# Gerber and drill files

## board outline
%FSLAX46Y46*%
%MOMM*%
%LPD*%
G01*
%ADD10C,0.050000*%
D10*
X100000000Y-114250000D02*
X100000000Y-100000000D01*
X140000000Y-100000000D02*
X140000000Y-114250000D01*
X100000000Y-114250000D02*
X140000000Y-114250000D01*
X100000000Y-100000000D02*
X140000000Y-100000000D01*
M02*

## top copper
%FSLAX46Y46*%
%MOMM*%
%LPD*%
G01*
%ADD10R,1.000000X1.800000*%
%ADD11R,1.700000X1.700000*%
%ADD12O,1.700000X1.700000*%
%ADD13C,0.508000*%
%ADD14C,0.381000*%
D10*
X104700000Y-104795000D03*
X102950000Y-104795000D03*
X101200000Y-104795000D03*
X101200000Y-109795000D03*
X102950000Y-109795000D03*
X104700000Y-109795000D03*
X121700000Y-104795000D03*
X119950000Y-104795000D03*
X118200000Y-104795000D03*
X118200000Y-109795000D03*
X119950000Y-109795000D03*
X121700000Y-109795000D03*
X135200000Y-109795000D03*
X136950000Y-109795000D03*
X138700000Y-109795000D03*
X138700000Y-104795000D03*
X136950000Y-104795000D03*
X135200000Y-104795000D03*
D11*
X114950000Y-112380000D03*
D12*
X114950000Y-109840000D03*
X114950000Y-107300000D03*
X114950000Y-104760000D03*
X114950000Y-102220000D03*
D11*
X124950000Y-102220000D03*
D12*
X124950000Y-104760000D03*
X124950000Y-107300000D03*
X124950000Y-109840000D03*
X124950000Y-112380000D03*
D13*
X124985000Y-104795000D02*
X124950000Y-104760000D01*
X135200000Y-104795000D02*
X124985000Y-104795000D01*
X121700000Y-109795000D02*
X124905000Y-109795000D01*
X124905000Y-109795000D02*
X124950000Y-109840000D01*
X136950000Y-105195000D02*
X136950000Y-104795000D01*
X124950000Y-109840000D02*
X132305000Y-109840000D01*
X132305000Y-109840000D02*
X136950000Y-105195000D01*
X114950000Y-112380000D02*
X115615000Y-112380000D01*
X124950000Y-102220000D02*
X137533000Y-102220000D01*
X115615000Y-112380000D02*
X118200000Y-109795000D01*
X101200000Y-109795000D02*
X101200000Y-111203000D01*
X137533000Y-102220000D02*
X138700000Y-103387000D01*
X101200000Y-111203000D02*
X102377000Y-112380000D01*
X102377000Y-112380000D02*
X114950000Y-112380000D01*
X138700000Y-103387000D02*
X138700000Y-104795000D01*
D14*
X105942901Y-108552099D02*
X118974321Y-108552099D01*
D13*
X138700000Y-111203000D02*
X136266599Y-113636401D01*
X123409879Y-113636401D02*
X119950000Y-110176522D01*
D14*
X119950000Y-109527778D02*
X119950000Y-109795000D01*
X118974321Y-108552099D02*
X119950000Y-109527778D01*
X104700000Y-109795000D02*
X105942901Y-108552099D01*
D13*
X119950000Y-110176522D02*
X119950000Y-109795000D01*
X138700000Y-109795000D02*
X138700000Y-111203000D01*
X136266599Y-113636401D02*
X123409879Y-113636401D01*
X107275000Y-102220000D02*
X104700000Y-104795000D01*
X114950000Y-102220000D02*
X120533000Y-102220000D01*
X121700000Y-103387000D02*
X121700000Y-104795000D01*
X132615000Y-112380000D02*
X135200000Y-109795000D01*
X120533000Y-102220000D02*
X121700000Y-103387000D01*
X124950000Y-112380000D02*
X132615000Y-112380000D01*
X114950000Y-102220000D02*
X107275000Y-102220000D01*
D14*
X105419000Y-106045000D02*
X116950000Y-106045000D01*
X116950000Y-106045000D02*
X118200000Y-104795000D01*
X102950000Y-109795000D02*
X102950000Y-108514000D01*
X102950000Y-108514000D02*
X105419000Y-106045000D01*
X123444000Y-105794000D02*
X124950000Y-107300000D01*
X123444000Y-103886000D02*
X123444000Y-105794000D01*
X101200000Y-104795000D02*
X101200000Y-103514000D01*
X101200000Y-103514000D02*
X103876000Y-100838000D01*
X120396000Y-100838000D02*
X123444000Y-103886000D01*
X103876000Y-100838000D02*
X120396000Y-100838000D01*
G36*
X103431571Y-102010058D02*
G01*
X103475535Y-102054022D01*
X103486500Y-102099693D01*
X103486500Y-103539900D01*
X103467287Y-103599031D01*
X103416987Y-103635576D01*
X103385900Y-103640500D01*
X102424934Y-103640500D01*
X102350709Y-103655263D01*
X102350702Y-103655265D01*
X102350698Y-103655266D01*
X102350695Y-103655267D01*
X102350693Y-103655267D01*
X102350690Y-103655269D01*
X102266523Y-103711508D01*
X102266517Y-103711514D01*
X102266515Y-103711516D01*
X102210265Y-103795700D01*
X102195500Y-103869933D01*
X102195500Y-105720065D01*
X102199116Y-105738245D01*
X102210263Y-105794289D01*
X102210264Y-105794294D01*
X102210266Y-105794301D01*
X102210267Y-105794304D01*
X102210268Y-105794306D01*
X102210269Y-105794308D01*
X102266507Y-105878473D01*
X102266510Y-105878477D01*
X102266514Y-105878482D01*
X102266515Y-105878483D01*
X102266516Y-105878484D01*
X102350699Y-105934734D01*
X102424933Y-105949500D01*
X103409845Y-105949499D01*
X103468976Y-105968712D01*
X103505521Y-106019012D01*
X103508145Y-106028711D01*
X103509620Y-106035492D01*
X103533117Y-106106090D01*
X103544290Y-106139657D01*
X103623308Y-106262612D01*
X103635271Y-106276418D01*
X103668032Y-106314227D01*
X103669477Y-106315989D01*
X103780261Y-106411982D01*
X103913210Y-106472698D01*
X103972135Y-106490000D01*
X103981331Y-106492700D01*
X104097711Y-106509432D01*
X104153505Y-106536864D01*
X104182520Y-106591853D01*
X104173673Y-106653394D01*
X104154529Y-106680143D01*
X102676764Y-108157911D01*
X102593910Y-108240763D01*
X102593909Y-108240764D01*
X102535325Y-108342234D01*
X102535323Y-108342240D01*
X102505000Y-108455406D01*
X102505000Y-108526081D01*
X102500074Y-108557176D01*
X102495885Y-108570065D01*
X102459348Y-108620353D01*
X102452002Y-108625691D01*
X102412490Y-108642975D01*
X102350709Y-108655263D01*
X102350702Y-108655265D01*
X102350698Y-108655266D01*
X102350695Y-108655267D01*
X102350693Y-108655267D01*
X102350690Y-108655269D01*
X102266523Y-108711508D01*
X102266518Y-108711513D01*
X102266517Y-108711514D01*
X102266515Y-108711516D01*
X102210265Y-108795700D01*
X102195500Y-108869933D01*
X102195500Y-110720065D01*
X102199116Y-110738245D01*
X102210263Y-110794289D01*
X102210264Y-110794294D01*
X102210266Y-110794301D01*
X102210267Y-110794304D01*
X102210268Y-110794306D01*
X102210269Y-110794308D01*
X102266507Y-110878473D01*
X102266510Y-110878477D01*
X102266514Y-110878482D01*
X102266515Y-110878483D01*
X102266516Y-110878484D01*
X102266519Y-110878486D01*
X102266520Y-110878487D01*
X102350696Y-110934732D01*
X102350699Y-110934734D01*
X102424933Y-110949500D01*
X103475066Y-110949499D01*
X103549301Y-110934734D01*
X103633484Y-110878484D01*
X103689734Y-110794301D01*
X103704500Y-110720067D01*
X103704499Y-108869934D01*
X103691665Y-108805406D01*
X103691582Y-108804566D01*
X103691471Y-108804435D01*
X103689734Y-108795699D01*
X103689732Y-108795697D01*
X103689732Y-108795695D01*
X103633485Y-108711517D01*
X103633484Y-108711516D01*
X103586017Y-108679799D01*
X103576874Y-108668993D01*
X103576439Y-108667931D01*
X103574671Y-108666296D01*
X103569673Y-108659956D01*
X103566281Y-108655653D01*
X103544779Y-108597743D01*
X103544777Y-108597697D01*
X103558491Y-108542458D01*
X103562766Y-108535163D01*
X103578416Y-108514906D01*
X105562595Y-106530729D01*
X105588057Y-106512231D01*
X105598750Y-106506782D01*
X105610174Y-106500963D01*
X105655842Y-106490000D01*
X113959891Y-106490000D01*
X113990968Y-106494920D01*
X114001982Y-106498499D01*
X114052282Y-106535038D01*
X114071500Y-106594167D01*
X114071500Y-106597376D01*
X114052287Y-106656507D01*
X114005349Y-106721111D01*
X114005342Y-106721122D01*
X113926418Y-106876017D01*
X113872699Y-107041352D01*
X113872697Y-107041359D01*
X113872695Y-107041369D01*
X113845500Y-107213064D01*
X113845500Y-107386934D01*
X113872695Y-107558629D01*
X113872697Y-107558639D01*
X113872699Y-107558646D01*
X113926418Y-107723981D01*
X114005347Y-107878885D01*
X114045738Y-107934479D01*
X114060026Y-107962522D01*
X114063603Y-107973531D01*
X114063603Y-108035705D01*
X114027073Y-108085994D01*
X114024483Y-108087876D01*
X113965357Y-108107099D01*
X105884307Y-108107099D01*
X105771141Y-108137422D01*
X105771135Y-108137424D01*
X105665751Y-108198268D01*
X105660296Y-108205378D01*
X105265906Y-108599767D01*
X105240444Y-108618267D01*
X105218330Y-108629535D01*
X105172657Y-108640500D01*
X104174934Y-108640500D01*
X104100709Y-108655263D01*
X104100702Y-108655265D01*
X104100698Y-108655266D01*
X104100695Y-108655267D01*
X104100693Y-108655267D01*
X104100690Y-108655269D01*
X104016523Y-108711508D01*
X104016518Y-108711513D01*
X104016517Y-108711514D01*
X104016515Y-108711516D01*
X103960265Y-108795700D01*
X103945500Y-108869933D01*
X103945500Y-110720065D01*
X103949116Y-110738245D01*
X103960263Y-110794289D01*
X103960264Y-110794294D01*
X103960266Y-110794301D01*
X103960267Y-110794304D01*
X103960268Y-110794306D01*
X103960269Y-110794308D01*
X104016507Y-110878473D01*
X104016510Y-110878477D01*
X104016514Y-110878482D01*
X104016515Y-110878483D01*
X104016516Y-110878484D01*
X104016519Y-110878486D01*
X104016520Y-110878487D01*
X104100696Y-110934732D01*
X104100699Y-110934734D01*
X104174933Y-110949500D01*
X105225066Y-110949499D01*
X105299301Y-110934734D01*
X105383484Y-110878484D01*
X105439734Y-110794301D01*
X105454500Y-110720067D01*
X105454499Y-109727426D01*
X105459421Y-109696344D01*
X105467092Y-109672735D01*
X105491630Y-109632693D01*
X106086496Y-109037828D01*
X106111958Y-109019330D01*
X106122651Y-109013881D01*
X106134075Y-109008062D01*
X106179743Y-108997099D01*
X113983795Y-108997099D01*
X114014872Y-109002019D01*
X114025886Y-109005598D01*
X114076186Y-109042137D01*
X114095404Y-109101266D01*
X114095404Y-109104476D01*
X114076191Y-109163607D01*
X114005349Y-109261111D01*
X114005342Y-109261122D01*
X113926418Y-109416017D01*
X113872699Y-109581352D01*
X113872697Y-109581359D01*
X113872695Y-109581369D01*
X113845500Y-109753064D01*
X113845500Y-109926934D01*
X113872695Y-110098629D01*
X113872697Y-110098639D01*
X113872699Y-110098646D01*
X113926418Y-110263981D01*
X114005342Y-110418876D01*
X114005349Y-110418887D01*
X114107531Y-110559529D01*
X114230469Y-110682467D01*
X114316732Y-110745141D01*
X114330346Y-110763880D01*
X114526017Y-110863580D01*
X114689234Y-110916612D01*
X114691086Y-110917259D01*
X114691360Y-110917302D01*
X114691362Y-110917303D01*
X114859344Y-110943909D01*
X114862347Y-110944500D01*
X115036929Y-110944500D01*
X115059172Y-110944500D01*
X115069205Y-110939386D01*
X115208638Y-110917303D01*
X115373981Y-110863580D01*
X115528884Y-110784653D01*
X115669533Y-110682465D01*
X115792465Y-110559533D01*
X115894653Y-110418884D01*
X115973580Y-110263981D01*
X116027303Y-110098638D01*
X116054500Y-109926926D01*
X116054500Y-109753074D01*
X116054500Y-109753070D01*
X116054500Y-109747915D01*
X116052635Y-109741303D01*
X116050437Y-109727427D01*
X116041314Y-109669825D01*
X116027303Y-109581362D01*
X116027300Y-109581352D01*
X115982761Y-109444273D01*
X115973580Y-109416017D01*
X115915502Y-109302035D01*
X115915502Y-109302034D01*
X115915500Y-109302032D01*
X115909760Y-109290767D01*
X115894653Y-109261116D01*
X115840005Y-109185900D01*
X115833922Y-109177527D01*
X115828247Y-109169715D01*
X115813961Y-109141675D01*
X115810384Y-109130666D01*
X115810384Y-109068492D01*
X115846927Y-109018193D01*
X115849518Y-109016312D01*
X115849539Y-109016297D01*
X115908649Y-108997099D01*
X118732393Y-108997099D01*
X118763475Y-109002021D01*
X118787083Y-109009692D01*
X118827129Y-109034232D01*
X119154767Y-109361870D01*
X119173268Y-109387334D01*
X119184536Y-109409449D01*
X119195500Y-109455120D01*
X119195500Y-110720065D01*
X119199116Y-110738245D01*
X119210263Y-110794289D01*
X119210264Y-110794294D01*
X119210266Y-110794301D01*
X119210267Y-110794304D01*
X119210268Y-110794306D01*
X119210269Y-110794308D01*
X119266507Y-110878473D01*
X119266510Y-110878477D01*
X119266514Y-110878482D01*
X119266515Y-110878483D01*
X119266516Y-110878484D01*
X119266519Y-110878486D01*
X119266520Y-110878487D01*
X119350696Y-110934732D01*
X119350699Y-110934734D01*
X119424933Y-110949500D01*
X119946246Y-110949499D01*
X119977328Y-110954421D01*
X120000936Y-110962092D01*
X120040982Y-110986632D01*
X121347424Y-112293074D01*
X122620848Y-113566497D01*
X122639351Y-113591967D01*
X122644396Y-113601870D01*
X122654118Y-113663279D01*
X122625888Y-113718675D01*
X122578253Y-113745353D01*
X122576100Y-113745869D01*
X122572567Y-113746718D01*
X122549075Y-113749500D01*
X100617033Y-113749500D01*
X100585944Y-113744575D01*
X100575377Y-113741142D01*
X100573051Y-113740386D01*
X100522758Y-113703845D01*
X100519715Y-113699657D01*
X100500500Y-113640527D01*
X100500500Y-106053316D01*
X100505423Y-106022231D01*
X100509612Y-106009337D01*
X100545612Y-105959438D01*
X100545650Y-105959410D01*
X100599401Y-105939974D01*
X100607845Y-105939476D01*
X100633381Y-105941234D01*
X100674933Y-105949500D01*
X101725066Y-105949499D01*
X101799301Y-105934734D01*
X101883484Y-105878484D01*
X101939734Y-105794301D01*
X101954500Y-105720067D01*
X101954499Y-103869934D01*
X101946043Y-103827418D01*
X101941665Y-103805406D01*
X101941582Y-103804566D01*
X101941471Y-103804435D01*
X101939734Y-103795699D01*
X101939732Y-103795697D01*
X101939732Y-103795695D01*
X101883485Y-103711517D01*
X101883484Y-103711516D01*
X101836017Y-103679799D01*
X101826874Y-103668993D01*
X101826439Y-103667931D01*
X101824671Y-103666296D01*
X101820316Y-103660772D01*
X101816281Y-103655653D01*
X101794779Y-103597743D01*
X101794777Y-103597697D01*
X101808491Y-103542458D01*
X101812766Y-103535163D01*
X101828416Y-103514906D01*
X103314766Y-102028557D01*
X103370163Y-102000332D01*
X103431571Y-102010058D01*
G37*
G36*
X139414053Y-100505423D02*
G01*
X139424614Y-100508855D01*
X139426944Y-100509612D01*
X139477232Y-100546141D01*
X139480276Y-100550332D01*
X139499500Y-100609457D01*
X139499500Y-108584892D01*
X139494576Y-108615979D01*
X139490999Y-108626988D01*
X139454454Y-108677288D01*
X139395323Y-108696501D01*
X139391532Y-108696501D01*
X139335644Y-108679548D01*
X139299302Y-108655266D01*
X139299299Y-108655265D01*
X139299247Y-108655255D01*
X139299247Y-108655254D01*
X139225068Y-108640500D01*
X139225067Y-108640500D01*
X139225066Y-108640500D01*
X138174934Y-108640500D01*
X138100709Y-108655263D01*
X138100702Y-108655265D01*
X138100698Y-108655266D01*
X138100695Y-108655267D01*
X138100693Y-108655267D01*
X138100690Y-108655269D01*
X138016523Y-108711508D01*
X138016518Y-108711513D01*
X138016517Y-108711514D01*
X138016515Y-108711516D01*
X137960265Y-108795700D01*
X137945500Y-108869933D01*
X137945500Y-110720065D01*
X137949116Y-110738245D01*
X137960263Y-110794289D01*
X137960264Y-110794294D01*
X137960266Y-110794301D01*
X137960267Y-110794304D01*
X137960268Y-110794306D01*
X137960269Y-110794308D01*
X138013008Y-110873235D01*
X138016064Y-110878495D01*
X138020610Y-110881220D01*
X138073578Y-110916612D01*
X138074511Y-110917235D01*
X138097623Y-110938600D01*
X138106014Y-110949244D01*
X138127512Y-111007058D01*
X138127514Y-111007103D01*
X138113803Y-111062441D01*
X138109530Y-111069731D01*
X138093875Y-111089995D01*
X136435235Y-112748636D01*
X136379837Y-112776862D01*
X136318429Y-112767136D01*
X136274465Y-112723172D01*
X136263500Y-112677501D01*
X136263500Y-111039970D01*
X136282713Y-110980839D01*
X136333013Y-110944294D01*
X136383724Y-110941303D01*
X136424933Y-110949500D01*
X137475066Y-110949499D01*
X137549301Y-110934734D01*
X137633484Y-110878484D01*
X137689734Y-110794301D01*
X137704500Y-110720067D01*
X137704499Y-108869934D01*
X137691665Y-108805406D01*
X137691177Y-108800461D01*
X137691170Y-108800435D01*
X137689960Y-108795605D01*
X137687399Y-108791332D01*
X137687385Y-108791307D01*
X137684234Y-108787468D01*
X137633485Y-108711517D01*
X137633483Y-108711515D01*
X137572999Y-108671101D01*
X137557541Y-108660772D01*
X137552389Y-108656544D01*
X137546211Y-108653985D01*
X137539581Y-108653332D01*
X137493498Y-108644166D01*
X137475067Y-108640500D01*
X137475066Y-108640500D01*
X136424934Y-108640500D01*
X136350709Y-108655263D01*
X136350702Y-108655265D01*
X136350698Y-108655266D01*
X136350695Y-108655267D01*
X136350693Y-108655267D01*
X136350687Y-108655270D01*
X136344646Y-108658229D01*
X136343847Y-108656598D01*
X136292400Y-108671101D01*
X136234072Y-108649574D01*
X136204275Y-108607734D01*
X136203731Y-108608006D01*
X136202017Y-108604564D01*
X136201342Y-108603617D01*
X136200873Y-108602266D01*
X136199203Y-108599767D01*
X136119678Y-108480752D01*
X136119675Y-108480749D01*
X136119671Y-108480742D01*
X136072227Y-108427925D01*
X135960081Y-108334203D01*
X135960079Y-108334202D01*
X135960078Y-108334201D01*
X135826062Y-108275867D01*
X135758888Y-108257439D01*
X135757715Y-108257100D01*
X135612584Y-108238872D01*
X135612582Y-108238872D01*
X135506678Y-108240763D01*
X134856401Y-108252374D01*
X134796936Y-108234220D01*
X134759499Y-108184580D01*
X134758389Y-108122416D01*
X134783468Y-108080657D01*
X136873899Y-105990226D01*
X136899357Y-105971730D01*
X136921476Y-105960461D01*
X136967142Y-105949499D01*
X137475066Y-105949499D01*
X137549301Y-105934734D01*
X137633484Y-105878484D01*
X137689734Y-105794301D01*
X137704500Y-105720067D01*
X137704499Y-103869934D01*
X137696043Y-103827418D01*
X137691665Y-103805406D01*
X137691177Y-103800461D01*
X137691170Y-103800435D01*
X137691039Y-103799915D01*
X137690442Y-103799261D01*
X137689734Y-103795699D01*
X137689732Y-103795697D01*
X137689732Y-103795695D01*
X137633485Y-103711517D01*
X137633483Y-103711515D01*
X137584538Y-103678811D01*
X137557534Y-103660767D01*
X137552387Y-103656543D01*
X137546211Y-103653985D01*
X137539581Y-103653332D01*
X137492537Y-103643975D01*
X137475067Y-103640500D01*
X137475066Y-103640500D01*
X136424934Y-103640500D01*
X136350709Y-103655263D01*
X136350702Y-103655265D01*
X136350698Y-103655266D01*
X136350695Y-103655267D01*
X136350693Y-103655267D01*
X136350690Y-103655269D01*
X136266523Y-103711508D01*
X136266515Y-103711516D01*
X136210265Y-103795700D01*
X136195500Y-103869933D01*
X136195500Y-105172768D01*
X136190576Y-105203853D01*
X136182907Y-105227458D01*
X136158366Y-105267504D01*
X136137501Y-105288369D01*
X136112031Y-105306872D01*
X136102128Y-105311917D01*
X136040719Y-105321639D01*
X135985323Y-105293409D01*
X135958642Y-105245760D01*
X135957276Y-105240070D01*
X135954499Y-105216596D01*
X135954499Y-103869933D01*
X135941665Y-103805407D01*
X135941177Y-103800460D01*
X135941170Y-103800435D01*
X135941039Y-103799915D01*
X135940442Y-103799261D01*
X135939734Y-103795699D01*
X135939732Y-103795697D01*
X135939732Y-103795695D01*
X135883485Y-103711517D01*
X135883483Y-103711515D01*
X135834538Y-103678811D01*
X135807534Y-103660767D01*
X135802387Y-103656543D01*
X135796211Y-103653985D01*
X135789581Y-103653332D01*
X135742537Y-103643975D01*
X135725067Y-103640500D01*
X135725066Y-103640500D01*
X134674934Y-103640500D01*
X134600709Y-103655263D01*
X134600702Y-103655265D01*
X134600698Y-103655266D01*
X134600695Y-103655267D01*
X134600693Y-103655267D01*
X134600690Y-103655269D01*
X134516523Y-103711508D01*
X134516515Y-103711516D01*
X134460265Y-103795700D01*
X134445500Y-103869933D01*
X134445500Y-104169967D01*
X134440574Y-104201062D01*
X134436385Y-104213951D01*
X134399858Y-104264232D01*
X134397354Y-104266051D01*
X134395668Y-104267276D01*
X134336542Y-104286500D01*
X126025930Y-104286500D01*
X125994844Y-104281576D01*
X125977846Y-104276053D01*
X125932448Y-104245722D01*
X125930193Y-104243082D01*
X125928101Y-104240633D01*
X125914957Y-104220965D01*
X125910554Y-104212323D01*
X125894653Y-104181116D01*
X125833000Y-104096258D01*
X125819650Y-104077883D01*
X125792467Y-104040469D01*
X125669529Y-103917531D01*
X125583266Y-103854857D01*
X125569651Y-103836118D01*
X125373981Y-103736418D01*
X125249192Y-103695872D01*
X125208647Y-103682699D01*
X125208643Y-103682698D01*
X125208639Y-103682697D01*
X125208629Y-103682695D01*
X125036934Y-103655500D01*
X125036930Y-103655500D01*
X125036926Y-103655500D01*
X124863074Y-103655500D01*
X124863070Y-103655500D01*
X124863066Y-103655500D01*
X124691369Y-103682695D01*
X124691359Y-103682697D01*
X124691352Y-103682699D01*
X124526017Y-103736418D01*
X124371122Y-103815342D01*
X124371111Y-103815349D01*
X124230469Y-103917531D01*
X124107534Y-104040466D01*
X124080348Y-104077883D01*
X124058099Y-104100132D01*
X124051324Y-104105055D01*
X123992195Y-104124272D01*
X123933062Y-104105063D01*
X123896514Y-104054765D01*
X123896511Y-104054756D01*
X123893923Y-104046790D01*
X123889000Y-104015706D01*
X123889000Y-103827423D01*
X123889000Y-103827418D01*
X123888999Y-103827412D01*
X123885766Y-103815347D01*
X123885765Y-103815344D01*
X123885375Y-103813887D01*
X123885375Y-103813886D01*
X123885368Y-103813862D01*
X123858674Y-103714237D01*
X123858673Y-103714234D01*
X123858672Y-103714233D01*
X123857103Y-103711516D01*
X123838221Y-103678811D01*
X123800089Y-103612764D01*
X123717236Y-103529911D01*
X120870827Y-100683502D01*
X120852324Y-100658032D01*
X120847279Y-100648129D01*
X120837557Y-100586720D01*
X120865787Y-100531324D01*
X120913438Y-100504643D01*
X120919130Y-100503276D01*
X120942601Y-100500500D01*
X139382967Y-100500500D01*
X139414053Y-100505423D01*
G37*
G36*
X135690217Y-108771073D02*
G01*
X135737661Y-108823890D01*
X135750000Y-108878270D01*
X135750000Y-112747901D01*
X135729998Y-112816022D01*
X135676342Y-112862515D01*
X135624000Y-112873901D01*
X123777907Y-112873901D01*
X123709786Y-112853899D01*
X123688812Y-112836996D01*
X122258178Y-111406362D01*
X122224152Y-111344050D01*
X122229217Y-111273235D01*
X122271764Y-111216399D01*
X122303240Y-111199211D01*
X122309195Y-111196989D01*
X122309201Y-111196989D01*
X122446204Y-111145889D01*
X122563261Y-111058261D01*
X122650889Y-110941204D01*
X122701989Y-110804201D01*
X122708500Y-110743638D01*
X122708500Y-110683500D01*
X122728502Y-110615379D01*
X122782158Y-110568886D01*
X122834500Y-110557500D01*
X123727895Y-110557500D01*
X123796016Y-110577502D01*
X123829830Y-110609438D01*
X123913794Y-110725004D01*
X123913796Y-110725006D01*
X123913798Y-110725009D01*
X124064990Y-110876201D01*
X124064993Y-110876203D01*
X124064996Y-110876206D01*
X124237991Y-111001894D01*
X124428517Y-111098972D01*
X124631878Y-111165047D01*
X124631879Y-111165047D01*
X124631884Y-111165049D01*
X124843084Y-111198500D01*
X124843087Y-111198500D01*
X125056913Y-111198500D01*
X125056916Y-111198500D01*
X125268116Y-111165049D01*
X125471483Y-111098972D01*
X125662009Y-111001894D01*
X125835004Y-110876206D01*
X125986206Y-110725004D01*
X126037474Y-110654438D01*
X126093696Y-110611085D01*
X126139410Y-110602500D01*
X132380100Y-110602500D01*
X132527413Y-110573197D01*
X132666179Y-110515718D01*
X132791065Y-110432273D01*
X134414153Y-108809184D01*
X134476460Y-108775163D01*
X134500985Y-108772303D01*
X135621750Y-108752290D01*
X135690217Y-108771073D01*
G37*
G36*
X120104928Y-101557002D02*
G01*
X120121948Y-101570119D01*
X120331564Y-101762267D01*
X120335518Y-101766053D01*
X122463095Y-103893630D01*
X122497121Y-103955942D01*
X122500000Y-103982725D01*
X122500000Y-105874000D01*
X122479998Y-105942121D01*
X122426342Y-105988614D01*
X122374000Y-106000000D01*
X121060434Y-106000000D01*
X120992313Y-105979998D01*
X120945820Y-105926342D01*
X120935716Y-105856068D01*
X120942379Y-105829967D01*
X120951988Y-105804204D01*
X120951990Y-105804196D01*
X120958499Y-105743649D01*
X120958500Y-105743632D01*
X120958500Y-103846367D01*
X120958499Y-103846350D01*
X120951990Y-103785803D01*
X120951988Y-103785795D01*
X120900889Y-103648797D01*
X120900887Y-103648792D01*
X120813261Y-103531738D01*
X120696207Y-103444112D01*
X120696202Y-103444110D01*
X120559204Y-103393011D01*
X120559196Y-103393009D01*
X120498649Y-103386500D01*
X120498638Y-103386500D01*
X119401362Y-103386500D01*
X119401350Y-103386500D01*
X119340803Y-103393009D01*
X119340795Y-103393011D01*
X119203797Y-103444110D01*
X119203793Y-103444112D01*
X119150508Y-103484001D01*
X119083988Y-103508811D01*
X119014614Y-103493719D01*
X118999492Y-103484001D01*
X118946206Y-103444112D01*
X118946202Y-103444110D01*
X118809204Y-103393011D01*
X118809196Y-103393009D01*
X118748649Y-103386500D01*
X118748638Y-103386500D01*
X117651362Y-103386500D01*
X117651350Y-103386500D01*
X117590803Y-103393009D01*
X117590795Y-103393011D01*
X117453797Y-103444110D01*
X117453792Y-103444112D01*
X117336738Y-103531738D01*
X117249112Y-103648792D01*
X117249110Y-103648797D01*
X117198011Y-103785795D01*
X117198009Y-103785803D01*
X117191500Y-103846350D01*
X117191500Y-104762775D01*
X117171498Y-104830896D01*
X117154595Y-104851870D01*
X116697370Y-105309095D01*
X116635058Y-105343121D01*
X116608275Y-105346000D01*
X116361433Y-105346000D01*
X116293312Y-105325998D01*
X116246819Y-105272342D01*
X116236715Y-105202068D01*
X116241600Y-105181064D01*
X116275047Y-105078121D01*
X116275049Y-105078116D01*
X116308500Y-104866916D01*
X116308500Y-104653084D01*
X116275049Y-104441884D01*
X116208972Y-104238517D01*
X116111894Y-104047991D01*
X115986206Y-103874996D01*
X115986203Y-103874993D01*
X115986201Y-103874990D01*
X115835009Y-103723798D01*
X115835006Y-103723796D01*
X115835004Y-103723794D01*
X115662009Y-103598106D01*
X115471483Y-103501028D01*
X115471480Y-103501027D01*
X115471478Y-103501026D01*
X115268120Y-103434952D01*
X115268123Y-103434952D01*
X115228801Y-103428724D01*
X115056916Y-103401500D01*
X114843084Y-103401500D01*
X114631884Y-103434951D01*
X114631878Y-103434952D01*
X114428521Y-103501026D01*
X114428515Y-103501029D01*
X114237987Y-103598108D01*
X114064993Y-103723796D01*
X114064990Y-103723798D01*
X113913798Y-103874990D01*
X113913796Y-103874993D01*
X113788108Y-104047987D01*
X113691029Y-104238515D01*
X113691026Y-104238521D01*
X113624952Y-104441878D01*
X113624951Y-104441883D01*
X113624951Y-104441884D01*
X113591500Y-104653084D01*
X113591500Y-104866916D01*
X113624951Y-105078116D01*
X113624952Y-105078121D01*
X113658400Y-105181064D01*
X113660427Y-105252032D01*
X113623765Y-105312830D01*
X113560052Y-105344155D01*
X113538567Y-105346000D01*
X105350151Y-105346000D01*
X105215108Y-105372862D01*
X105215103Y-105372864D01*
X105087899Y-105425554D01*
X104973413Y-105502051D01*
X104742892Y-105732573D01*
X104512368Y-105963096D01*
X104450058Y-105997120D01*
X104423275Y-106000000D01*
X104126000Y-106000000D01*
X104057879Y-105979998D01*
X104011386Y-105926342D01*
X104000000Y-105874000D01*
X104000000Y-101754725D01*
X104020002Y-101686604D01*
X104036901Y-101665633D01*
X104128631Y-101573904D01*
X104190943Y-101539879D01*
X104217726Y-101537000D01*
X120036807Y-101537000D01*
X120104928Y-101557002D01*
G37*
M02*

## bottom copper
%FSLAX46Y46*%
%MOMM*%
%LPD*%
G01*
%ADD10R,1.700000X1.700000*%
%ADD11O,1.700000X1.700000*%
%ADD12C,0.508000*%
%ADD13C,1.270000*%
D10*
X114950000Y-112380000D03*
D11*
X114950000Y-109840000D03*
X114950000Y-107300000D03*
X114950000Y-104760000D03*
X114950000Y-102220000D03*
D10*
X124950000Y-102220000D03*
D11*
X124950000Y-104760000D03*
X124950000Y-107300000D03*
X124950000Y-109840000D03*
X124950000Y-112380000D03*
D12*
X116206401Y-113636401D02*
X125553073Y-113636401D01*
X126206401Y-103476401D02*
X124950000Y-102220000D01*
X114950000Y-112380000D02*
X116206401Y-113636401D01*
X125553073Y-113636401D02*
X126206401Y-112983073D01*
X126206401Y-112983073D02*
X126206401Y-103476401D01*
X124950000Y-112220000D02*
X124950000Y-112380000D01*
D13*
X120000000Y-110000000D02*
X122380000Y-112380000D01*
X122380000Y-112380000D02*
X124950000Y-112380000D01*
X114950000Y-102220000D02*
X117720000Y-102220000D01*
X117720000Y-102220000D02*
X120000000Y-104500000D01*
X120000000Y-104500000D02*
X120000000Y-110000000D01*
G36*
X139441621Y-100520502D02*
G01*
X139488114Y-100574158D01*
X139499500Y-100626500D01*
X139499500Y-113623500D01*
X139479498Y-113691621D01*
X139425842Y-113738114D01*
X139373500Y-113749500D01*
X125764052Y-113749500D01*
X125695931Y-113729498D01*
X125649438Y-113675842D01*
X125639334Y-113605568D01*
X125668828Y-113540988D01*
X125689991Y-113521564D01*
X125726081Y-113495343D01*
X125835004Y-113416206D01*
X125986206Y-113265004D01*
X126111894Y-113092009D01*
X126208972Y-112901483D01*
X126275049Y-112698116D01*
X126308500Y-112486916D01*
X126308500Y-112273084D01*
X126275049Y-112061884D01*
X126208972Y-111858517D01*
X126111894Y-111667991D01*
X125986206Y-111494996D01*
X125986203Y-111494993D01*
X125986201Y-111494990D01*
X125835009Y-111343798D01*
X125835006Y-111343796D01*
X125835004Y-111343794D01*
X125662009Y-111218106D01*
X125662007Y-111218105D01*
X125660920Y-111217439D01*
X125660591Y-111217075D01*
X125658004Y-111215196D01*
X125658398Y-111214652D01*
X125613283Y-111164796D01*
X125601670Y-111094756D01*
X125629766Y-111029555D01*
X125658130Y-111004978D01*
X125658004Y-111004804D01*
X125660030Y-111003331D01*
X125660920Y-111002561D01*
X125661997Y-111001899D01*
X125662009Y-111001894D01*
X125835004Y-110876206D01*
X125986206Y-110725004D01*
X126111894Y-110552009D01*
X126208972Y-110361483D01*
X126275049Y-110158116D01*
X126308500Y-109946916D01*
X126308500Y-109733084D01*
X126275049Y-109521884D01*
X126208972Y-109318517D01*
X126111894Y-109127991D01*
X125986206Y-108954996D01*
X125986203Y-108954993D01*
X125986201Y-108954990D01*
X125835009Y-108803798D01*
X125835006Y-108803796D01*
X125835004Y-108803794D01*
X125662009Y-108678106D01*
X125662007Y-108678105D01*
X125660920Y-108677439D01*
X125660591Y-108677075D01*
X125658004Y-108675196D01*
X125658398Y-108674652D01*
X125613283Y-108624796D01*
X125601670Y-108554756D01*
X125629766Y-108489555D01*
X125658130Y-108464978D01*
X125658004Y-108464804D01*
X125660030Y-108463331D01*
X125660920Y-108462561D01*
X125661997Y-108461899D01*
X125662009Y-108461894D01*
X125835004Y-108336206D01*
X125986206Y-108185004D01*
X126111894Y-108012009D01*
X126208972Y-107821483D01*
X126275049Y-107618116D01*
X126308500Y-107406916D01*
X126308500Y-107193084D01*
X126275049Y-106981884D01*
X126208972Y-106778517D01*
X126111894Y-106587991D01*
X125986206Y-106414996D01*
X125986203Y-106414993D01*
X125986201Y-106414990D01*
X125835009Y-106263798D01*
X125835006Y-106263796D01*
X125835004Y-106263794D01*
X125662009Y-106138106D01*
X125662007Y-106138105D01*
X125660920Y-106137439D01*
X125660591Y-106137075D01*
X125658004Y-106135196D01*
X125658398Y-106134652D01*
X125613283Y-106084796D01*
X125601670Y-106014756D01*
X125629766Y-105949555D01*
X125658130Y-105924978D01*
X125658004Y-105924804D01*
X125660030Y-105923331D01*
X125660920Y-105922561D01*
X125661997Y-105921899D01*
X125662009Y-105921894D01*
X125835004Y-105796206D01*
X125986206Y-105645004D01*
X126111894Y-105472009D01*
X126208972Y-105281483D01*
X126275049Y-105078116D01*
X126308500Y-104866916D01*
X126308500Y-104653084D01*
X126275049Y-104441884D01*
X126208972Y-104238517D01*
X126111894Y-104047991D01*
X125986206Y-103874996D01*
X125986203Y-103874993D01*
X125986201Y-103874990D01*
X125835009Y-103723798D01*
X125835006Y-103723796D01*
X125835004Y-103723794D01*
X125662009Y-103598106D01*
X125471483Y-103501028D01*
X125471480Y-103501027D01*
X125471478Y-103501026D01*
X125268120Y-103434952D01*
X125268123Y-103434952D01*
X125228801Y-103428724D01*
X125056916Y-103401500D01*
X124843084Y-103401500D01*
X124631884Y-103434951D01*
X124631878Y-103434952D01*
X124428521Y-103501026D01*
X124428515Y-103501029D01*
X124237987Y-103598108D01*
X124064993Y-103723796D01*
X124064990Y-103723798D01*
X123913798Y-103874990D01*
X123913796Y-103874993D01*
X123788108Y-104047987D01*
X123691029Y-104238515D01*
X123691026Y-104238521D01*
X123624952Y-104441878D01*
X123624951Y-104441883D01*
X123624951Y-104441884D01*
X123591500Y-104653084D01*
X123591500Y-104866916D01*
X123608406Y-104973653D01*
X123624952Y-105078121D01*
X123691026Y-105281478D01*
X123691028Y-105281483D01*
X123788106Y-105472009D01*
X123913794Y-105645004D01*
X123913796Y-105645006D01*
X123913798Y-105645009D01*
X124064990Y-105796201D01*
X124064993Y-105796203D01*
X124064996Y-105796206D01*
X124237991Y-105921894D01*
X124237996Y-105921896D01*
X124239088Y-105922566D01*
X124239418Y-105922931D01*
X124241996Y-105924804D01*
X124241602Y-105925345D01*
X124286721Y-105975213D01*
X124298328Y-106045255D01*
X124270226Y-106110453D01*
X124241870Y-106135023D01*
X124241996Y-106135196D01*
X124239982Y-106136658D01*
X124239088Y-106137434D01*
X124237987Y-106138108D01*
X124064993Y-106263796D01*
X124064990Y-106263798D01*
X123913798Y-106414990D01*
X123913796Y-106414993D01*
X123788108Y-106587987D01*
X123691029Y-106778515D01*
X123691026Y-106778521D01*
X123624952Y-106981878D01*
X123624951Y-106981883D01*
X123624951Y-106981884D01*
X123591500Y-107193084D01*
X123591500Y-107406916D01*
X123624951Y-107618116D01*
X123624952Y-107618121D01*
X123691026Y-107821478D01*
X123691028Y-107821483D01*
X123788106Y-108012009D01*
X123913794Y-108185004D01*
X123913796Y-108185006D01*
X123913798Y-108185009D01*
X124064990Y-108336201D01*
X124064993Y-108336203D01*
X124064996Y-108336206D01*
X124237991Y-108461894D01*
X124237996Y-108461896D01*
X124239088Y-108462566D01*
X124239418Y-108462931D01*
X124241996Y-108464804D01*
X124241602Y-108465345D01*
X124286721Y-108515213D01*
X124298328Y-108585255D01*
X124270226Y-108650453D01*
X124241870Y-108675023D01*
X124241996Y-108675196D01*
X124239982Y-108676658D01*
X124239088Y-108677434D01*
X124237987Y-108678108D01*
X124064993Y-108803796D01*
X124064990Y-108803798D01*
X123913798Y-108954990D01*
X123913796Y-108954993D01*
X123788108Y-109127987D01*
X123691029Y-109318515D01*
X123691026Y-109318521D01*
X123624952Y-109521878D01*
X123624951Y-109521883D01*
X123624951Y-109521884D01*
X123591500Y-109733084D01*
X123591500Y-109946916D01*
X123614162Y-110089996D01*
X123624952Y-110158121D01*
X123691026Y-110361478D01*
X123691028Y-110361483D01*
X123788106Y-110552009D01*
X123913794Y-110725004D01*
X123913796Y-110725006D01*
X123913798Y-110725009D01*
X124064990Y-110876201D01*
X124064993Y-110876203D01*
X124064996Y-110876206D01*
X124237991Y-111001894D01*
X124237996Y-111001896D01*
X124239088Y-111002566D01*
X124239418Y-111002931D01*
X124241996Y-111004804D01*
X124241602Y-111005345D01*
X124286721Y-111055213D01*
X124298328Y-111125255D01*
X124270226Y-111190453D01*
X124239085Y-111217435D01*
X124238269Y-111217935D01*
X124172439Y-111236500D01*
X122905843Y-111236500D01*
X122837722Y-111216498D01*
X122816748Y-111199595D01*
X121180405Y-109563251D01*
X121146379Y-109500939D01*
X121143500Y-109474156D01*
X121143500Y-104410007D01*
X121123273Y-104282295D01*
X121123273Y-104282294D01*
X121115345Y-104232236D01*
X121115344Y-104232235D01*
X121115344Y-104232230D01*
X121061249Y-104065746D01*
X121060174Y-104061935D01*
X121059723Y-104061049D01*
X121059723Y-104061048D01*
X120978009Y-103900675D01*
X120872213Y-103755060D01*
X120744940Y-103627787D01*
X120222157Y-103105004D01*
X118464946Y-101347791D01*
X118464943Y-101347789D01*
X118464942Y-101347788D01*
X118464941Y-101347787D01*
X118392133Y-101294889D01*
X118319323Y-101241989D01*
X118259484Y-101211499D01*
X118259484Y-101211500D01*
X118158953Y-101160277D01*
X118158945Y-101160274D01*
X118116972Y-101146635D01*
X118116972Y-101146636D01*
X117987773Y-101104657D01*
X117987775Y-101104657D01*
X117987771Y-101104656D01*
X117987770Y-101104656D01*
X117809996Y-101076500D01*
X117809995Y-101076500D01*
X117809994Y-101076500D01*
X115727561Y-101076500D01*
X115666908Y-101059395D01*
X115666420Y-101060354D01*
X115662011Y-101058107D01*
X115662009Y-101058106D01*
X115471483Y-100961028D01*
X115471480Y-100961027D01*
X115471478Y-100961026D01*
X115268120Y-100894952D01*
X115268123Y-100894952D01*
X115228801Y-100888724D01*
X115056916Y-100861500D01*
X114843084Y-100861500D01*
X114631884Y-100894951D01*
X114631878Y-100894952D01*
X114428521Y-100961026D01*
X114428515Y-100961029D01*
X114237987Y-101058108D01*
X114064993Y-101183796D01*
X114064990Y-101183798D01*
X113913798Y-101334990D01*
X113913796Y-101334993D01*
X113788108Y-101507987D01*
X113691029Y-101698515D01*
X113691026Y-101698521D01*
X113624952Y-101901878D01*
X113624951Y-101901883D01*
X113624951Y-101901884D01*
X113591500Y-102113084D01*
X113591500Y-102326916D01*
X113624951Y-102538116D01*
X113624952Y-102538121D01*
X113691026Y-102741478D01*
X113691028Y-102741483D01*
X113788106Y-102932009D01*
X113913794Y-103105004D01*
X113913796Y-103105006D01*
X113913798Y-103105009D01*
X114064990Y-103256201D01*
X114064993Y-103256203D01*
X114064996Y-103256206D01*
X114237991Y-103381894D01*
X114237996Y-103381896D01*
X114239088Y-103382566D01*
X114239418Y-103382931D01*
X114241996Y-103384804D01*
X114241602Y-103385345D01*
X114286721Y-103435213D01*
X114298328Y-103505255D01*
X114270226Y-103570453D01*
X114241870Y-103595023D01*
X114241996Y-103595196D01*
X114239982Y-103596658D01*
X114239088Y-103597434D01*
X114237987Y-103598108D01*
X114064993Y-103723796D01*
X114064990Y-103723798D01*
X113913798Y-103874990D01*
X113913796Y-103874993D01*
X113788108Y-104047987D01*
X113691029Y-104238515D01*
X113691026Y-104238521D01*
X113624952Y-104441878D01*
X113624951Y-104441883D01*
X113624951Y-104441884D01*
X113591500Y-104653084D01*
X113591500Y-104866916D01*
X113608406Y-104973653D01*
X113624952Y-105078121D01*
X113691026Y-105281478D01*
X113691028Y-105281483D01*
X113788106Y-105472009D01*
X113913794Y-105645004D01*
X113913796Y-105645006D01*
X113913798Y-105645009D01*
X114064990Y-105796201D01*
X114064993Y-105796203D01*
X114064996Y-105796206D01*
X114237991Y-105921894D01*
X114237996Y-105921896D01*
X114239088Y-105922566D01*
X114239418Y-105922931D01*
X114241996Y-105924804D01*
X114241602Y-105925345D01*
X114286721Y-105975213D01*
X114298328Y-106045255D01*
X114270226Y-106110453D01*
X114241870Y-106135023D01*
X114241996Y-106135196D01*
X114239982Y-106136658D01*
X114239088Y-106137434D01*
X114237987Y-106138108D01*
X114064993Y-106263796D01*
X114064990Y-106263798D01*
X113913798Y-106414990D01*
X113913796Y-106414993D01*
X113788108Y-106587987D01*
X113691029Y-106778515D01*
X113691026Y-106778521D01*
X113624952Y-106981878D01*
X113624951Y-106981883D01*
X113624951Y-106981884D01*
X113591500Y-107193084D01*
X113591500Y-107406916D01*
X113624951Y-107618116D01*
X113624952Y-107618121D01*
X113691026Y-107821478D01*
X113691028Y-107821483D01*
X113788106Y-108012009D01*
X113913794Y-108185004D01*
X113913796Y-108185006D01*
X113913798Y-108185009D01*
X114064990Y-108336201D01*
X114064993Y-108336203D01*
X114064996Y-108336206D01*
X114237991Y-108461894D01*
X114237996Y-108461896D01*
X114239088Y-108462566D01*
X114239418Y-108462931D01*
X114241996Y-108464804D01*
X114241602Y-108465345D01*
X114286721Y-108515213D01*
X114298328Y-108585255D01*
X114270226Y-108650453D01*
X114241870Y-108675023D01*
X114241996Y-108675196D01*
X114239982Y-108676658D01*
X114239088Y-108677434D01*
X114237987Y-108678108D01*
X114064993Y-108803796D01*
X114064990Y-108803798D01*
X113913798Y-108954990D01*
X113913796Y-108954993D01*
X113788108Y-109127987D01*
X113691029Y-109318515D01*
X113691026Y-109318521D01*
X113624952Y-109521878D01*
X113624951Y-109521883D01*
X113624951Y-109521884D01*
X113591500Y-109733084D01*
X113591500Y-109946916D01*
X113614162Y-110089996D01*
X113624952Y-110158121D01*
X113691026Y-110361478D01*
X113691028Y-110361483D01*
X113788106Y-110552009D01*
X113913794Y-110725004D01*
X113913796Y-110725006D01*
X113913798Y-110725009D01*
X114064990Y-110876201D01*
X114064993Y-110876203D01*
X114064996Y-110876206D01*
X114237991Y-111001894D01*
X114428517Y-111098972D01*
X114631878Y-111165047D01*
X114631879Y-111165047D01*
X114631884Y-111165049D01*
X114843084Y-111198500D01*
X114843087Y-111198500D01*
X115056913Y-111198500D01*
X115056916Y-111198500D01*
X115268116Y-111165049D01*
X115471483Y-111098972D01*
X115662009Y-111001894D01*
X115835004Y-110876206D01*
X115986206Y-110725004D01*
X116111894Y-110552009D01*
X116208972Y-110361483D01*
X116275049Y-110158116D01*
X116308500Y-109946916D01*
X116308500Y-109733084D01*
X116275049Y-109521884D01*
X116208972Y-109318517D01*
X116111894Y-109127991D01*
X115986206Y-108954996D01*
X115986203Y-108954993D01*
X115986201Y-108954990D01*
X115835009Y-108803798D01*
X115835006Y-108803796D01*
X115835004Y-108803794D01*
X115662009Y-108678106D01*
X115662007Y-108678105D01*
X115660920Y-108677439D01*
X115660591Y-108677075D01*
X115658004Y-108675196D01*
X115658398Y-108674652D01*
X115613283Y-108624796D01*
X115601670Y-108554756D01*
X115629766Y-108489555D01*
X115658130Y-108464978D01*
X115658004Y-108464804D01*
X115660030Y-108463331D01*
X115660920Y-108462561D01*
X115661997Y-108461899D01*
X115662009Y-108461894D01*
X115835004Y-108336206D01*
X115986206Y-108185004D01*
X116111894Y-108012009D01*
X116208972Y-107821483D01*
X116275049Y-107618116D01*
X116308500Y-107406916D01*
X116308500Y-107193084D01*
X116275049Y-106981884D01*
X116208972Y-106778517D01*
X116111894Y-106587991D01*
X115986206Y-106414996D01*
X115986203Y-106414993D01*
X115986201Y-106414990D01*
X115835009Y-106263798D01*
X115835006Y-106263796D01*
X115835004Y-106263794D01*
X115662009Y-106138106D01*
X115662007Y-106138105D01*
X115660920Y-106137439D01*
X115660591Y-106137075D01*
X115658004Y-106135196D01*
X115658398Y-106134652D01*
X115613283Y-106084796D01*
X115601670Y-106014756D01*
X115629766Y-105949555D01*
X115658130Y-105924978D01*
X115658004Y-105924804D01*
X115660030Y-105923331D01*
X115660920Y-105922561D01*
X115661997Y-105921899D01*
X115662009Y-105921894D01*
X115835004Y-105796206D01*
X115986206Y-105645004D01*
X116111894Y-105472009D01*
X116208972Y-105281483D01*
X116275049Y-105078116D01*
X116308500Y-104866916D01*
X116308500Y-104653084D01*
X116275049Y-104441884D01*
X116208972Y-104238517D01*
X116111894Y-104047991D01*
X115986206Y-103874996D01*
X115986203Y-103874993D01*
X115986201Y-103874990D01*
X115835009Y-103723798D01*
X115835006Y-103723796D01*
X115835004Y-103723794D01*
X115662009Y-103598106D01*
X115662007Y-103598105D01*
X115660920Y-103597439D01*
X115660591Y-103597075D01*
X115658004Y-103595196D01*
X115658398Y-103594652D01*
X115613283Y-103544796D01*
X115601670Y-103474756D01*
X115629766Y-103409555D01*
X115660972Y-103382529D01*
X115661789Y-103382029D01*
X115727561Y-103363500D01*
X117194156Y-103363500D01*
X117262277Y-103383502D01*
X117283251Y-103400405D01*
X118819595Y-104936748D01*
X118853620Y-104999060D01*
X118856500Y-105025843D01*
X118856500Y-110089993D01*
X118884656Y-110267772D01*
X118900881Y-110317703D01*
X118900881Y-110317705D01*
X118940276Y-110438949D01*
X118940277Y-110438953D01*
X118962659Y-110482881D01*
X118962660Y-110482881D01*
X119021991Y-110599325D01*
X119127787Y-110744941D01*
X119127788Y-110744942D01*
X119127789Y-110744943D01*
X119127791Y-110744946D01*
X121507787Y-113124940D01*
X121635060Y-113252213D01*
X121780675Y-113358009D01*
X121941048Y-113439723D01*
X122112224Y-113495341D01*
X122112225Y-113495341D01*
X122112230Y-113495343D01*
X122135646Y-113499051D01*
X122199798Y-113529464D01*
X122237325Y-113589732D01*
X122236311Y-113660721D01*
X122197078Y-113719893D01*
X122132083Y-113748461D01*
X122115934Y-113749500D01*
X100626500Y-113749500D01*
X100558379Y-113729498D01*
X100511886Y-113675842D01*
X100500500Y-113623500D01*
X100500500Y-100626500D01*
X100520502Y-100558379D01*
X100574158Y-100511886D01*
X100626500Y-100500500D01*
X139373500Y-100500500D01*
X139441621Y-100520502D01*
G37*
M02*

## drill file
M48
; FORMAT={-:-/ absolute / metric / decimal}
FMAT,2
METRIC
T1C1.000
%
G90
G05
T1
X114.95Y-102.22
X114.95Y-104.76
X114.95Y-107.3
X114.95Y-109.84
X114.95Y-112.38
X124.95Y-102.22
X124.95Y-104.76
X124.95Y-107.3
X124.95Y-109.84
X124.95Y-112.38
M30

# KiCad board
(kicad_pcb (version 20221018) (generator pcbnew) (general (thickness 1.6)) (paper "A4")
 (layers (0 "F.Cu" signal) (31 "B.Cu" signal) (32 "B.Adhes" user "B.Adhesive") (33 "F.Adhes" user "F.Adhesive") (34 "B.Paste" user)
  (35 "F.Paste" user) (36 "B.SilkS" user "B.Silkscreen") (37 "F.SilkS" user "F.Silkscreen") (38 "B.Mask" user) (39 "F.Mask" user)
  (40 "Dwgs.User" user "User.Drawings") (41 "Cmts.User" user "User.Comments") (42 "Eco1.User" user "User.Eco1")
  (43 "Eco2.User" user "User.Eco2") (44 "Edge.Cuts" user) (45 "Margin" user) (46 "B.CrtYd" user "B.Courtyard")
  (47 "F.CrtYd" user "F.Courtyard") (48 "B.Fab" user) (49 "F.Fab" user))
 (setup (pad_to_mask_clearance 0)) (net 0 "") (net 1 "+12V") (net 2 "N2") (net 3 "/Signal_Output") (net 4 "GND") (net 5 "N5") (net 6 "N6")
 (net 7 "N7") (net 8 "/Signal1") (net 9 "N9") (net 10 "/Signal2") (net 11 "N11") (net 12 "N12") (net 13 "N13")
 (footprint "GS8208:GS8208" (layer "F.Cu") (at 102.95 107.295 -90)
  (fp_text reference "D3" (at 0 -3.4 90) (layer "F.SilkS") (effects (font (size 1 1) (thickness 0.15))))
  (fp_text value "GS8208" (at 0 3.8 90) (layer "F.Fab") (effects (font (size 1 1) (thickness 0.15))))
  (pad "1" smd rect (at -2.5 -1.75 270) (size 1.8 1) (layers "F.Cu" "F.Paste" "F.Mask") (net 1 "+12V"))
  (pad "2" smd rect (at -2.5 0 270) (size 1.8 1) (layers "F.Cu" "F.Paste" "F.Mask") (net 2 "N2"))
  (pad "3" smd rect (at -2.5 1.75 270) (size 1.8 1) (layers "F.Cu" "F.Paste" "F.Mask") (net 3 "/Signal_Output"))
  (pad "4" smd rect (at 2.5 1.75 270) (size 1.8 1) (layers "F.Cu" "F.Paste" "F.Mask") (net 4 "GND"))
  (pad "5" smd rect (at 2.5 0 270) (size 1.8 1) (layers "F.Cu" "F.Paste" "F.Mask") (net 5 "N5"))
  (pad "6" smd rect (at 2.5 -1.75 270) (size 1.8 1) (layers "F.Cu" "F.Paste" "F.Mask") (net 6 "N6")))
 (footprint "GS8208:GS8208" (layer "F.Cu") (at 119.95 107.295 -90)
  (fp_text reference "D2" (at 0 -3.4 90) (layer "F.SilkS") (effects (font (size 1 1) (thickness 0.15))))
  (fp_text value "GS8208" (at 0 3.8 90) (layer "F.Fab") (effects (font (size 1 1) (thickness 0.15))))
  (pad "1" smd rect (at -2.5 -1.75 270) (size 1.8 1) (layers "F.Cu" "F.Paste" "F.Mask") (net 1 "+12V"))
  (pad "2" smd rect (at -2.5 0 270) (size 1.8 1) (layers "F.Cu" "F.Paste" "F.Mask") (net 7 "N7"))
  (pad "3" smd rect (at -2.5 1.75 270) (size 1.8 1) (layers "F.Cu" "F.Paste" "F.Mask") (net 5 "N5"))
  (pad "4" smd rect (at 2.5 1.75 270) (size 1.8 1) (layers "F.Cu" "F.Paste" "F.Mask") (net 4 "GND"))
  (pad "5" smd rect (at 2.5 0 270) (size 1.8 1) (layers "F.Cu" "F.Paste" "F.Mask") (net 6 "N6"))
  (pad "6" smd rect (at 2.5 -1.75 270) (size 1.8 1) (layers "F.Cu" "F.Paste" "F.Mask") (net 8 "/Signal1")))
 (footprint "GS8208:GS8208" (layer "F.Cu") (at 136.95 107.295 90)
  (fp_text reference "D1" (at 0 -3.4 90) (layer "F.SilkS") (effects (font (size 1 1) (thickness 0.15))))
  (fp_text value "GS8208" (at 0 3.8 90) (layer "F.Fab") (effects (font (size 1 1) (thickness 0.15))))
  (pad "1" smd rect (at -2.5 -1.75 90) (size 1.8 1) (layers "F.Cu" "F.Paste" "F.Mask") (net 1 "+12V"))
  (pad "2" smd rect (at -2.5 0 90) (size 1.8 1) (layers "F.Cu" "F.Paste" "F.Mask") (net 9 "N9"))
  (pad "3" smd rect (at -2.5 1.75 90) (size 1.8 1) (layers "F.Cu" "F.Paste" "F.Mask") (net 6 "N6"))
  (pad "4" smd rect (at 2.5 1.75 90) (size 1.8 1) (layers "F.Cu" "F.Paste" "F.Mask") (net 4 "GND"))
  (pad "5" smd rect (at 2.5 0 90) (size 1.8 1) (layers "F.Cu" "F.Paste" "F.Mask") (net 8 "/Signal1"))
  (pad "6" smd rect (at 2.5 -1.75 90) (size 1.8 1) (layers "F.Cu" "F.Paste" "F.Mask") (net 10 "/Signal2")))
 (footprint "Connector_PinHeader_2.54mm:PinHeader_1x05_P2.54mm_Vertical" (layer "B.Cu") (at 114.95 112.38)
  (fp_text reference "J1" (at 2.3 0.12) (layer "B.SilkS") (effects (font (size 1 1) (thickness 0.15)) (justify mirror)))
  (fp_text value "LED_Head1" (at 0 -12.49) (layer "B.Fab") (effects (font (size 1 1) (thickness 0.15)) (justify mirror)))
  (pad "1" thru_hole rect (at 0 0) (size 1.7 1.7) (drill 1) (layers "*.Cu" "*.Mask") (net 4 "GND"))
  (pad "2" thru_hole oval (at 0 -2.54) (size 1.7 1.7) (drill 1) (layers "*.Cu" "*.Mask") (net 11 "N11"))
  (pad "3" thru_hole oval (at 0 -5.08) (size 1.7 1.7) (drill 1) (layers "*.Cu" "*.Mask") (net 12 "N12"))
  (pad "4" thru_hole oval (at 0 -7.62) (size 1.7 1.7) (drill 1) (layers "*.Cu" "*.Mask") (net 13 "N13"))
  (pad "5" thru_hole oval (at 0 -10.16) (size 1.7 1.7) (drill 1) (layers "*.Cu" "*.Mask") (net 1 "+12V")))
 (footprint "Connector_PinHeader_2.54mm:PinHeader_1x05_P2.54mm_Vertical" (layer "B.Cu") (at 124.95 102.22 180)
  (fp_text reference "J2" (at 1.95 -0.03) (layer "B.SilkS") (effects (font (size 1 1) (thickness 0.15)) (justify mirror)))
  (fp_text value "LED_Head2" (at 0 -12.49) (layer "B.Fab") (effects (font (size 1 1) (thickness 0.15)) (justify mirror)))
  (pad "1" thru_hole rect (at 0 0 180) (size 1.7 1.7) (drill 1) (layers "*.Cu" "*.Mask") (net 4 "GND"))
  (pad "2" thru_hole oval (at 0 -2.54 180) (size 1.7 1.7) (drill 1) (layers "*.Cu" "*.Mask") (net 10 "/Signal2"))
  (pad "3" thru_hole oval (at 0 -5.08 180) (size 1.7 1.7) (drill 1) (layers "*.Cu" "*.Mask") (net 3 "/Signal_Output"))
  (pad "4" thru_hole oval (at 0 -7.62 180) (size 1.7 1.7) (drill 1) (layers "*.Cu" "*.Mask") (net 8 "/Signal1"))
  (pad "5" thru_hole oval (at 0 -10.16 180) (size 1.7 1.7) (drill 1) (layers "*.Cu" "*.Mask") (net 1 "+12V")))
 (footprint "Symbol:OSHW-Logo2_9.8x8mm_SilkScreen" (layer "B.Cu") (at 132.5 107 180)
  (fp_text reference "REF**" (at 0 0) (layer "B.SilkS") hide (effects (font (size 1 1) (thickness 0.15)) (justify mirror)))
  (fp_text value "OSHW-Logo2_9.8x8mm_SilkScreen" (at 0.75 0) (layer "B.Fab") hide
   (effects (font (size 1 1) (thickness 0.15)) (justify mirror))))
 (gr_line (start 100 114.25) (end 100 100) (stroke (width 0.05) (type solid)) (layer "Edge.Cuts"))
 (gr_line (start 140 100) (end 140 114.25) (stroke (width 0.05) (type solid)) (layer "Edge.Cuts"))
 (gr_line (start 100 114.25) (end 140 114.25) (stroke (width 0.05) (type solid)) (layer "Edge.Cuts"))
 (gr_line (start 100 100) (end 140 100) (stroke (width 0.05) (type solid)) (layer "Edge.Cuts"))
 (segment (start 124.985 104.795) (end 124.95 104.76) (width 0.508) (layer "F.Cu") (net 10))
 (segment (start 135.2 104.795) (end 124.985 104.795) (width 0.508) (layer "F.Cu") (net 10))
 (segment (start 121.7 109.795) (end 124.905 109.795) (width 0.508) (layer "F.Cu") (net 8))
 (segment (start 124.905 109.795) (end 124.95 109.84) (width 0.508) (layer "F.Cu") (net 8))
 (segment (start 136.95 105.195) (end 136.95 104.795) (width 0.508) (layer "F.Cu") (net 8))
 (segment (start 124.95 109.84) (end 132.305 109.84) (width 0.508) (layer "F.Cu") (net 8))
 (segment (start 132.305 109.84) (end 136.95 105.195) (width 0.508) (layer "F.Cu") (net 8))
 (segment (start 114.95 112.38) (end 115.615 112.38) (width 0.508) (layer "F.Cu") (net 4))
 (segment (start 124.95 102.22) (end 137.533 102.22) (width 0.508) (layer "F.Cu") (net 4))
 (segment (start 115.615 112.38) (end 118.2 109.795) (width 0.508) (layer "F.Cu") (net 4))
 (segment (start 101.2 109.795) (end 101.2 111.203) (width 0.508) (layer "F.Cu") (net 4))
 (segment (start 137.533 102.22) (end 138.7 103.387) (width 0.508) (layer "F.Cu") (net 4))
 (segment (start 101.2 111.203) (end 102.377 112.38) (width 0.508) (layer "F.Cu") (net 4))
 (segment (start 102.377 112.38) (end 114.95 112.38) (width 0.508) (layer "F.Cu") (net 4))
 (segment (start 138.7 103.387) (end 138.7 104.795) (width 0.508) (layer "F.Cu") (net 4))
 (segment (start 116.206401 113.636401) (end 125.553073 113.636401) (width 0.508) (layer "B.Cu") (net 4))
 (segment (start 126.206401 103.476401) (end 124.95 102.22) (width 0.508) (layer "B.Cu") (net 4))
 (segment (start 114.95 112.38) (end 116.206401 113.636401) (width 0.508) (layer "B.Cu") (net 4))
 (segment (start 125.553073 113.636401) (end 126.206401 112.983073) (width 0.508) (layer "B.Cu") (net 4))
 (segment (start 126.206401 112.983073) (end 126.206401 103.476401) (width 0.508) (layer "B.Cu") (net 4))
 (segment (start 105.942901 108.552099) (end 118.974321 108.552099) (width 0.381) (layer "F.Cu") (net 6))
 (segment (start 138.7 111.203) (end 136.266599 113.636401) (width 0.508) (layer "F.Cu") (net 6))
 (segment (start 123.409879 113.636401) (end 119.95 110.176522) (width 0.508) (layer "F.Cu") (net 6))
 (segment (start 119.95 109.527778) (end 119.95 109.795) (width 0.381) (layer "F.Cu") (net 6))
 (segment (start 118.974321 108.552099) (end 119.95 109.527778) (width 0.381) (layer "F.Cu") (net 6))
 (segment (start 104.7 109.795) (end 105.942901 108.552099) (width 0.381) (layer "F.Cu") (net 6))
 (segment (start 119.95 110.176522) (end 119.95 109.795) (width 0.508) (layer "F.Cu") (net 6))
 (segment (start 138.7 109.795) (end 138.7 111.203) (width 0.508) (layer "F.Cu") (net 6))
 (segment (start 136.266599 113.636401) (end 123.409879 113.636401) (width 0.508) (layer "F.Cu") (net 6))
 (segment (start 107.275 102.22) (end 104.7 104.795) (width 0.508) (layer "F.Cu") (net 1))
 (segment (start 114.95 102.22) (end 120.533 102.22) (width 0.508) (layer "F.Cu") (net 1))
 (segment (start 121.7 103.387) (end 121.7 104.795) (width 0.508) (layer "F.Cu") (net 1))
 (segment (start 132.615 112.38) (end 135.2 109.795) (width 0.508) (layer "F.Cu") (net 1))
 (segment (start 120.533 102.22) (end 121.7 103.387) (width 0.508) (layer "F.Cu") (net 1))
 (segment (start 124.95 112.38) (end 132.615 112.38) (width 0.508) (layer "F.Cu") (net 1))
 (segment (start 114.95 102.22) (end 107.275 102.22) (width 0.508) (layer "F.Cu") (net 1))
 (segment (start 124.95 112.22) (end 124.95 112.38) (width 0.508) (layer "B.Cu") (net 1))
 (segment (start 120 110) (end 122.38 112.38) (width 1.27) (layer "B.Cu") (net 1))
 (segment (start 122.38 112.38) (end 124.95 112.38) (width 1.27) (layer "B.Cu") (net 1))
 (segment (start 114.95 102.22) (end 117.72 102.22) (width 1.27) (layer "B.Cu") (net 1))
 (segment (start 117.72 102.22) (end 120 104.5) (width 1.27) (layer "B.Cu") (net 1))
 (segment (start 120 104.5) (end 120 110) (width 1.27) (layer "B.Cu") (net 1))
 (segment (start 105.419 106.045) (end 116.95 106.045) (width 0.381) (layer "F.Cu") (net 5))
 (segment (start 116.95 106.045) (end 118.2 104.795) (width 0.381) (layer "F.Cu") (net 5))
 (segment (start 102.95 109.795) (end 102.95 108.514) (width 0.381) (layer "F.Cu") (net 5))
 (segment (start 102.95 108.514) (end 105.419 106.045) (width 0.381) (layer "F.Cu") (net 5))
 (segment (start 123.444 105.794) (end 124.95 107.3) (width 0.381) (layer "F.Cu") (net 3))
 (segment (start 123.444 103.886) (end 123.444 105.794) (width 0.381) (layer "F.Cu") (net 3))
 (segment (start 101.2 104.795) (end 101.2 103.514) (width 0.381) (layer "F.Cu") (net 3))
 (segment (start 101.2 103.514) (end 103.876 100.838) (width 0.381) (layer "F.Cu") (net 3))
 (segment (start 120.396 100.838) (end 123.444 103.886) (width 0.381) (layer "F.Cu") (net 3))
 (segment (start 103.876 100.838) (end 120.396 100.838) (width 0.381) (layer "F.Cu") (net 3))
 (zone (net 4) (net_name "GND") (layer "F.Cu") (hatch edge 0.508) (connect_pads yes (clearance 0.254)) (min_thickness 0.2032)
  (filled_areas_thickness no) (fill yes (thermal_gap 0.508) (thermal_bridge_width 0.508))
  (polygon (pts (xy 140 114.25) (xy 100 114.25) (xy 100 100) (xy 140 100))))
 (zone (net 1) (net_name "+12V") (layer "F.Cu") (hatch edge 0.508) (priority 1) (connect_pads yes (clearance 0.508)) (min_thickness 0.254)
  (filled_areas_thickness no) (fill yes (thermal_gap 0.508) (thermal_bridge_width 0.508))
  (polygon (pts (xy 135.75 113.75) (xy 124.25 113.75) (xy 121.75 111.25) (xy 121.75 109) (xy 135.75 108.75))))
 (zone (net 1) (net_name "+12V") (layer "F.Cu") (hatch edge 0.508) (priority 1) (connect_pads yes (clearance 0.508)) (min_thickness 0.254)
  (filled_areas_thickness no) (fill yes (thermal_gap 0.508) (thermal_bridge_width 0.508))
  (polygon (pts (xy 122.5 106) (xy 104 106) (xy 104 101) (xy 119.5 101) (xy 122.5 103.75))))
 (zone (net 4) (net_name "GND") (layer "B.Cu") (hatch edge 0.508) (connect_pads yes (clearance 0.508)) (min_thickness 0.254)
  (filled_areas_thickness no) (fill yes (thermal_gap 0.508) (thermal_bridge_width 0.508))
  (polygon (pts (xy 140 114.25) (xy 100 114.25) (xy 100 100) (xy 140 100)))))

